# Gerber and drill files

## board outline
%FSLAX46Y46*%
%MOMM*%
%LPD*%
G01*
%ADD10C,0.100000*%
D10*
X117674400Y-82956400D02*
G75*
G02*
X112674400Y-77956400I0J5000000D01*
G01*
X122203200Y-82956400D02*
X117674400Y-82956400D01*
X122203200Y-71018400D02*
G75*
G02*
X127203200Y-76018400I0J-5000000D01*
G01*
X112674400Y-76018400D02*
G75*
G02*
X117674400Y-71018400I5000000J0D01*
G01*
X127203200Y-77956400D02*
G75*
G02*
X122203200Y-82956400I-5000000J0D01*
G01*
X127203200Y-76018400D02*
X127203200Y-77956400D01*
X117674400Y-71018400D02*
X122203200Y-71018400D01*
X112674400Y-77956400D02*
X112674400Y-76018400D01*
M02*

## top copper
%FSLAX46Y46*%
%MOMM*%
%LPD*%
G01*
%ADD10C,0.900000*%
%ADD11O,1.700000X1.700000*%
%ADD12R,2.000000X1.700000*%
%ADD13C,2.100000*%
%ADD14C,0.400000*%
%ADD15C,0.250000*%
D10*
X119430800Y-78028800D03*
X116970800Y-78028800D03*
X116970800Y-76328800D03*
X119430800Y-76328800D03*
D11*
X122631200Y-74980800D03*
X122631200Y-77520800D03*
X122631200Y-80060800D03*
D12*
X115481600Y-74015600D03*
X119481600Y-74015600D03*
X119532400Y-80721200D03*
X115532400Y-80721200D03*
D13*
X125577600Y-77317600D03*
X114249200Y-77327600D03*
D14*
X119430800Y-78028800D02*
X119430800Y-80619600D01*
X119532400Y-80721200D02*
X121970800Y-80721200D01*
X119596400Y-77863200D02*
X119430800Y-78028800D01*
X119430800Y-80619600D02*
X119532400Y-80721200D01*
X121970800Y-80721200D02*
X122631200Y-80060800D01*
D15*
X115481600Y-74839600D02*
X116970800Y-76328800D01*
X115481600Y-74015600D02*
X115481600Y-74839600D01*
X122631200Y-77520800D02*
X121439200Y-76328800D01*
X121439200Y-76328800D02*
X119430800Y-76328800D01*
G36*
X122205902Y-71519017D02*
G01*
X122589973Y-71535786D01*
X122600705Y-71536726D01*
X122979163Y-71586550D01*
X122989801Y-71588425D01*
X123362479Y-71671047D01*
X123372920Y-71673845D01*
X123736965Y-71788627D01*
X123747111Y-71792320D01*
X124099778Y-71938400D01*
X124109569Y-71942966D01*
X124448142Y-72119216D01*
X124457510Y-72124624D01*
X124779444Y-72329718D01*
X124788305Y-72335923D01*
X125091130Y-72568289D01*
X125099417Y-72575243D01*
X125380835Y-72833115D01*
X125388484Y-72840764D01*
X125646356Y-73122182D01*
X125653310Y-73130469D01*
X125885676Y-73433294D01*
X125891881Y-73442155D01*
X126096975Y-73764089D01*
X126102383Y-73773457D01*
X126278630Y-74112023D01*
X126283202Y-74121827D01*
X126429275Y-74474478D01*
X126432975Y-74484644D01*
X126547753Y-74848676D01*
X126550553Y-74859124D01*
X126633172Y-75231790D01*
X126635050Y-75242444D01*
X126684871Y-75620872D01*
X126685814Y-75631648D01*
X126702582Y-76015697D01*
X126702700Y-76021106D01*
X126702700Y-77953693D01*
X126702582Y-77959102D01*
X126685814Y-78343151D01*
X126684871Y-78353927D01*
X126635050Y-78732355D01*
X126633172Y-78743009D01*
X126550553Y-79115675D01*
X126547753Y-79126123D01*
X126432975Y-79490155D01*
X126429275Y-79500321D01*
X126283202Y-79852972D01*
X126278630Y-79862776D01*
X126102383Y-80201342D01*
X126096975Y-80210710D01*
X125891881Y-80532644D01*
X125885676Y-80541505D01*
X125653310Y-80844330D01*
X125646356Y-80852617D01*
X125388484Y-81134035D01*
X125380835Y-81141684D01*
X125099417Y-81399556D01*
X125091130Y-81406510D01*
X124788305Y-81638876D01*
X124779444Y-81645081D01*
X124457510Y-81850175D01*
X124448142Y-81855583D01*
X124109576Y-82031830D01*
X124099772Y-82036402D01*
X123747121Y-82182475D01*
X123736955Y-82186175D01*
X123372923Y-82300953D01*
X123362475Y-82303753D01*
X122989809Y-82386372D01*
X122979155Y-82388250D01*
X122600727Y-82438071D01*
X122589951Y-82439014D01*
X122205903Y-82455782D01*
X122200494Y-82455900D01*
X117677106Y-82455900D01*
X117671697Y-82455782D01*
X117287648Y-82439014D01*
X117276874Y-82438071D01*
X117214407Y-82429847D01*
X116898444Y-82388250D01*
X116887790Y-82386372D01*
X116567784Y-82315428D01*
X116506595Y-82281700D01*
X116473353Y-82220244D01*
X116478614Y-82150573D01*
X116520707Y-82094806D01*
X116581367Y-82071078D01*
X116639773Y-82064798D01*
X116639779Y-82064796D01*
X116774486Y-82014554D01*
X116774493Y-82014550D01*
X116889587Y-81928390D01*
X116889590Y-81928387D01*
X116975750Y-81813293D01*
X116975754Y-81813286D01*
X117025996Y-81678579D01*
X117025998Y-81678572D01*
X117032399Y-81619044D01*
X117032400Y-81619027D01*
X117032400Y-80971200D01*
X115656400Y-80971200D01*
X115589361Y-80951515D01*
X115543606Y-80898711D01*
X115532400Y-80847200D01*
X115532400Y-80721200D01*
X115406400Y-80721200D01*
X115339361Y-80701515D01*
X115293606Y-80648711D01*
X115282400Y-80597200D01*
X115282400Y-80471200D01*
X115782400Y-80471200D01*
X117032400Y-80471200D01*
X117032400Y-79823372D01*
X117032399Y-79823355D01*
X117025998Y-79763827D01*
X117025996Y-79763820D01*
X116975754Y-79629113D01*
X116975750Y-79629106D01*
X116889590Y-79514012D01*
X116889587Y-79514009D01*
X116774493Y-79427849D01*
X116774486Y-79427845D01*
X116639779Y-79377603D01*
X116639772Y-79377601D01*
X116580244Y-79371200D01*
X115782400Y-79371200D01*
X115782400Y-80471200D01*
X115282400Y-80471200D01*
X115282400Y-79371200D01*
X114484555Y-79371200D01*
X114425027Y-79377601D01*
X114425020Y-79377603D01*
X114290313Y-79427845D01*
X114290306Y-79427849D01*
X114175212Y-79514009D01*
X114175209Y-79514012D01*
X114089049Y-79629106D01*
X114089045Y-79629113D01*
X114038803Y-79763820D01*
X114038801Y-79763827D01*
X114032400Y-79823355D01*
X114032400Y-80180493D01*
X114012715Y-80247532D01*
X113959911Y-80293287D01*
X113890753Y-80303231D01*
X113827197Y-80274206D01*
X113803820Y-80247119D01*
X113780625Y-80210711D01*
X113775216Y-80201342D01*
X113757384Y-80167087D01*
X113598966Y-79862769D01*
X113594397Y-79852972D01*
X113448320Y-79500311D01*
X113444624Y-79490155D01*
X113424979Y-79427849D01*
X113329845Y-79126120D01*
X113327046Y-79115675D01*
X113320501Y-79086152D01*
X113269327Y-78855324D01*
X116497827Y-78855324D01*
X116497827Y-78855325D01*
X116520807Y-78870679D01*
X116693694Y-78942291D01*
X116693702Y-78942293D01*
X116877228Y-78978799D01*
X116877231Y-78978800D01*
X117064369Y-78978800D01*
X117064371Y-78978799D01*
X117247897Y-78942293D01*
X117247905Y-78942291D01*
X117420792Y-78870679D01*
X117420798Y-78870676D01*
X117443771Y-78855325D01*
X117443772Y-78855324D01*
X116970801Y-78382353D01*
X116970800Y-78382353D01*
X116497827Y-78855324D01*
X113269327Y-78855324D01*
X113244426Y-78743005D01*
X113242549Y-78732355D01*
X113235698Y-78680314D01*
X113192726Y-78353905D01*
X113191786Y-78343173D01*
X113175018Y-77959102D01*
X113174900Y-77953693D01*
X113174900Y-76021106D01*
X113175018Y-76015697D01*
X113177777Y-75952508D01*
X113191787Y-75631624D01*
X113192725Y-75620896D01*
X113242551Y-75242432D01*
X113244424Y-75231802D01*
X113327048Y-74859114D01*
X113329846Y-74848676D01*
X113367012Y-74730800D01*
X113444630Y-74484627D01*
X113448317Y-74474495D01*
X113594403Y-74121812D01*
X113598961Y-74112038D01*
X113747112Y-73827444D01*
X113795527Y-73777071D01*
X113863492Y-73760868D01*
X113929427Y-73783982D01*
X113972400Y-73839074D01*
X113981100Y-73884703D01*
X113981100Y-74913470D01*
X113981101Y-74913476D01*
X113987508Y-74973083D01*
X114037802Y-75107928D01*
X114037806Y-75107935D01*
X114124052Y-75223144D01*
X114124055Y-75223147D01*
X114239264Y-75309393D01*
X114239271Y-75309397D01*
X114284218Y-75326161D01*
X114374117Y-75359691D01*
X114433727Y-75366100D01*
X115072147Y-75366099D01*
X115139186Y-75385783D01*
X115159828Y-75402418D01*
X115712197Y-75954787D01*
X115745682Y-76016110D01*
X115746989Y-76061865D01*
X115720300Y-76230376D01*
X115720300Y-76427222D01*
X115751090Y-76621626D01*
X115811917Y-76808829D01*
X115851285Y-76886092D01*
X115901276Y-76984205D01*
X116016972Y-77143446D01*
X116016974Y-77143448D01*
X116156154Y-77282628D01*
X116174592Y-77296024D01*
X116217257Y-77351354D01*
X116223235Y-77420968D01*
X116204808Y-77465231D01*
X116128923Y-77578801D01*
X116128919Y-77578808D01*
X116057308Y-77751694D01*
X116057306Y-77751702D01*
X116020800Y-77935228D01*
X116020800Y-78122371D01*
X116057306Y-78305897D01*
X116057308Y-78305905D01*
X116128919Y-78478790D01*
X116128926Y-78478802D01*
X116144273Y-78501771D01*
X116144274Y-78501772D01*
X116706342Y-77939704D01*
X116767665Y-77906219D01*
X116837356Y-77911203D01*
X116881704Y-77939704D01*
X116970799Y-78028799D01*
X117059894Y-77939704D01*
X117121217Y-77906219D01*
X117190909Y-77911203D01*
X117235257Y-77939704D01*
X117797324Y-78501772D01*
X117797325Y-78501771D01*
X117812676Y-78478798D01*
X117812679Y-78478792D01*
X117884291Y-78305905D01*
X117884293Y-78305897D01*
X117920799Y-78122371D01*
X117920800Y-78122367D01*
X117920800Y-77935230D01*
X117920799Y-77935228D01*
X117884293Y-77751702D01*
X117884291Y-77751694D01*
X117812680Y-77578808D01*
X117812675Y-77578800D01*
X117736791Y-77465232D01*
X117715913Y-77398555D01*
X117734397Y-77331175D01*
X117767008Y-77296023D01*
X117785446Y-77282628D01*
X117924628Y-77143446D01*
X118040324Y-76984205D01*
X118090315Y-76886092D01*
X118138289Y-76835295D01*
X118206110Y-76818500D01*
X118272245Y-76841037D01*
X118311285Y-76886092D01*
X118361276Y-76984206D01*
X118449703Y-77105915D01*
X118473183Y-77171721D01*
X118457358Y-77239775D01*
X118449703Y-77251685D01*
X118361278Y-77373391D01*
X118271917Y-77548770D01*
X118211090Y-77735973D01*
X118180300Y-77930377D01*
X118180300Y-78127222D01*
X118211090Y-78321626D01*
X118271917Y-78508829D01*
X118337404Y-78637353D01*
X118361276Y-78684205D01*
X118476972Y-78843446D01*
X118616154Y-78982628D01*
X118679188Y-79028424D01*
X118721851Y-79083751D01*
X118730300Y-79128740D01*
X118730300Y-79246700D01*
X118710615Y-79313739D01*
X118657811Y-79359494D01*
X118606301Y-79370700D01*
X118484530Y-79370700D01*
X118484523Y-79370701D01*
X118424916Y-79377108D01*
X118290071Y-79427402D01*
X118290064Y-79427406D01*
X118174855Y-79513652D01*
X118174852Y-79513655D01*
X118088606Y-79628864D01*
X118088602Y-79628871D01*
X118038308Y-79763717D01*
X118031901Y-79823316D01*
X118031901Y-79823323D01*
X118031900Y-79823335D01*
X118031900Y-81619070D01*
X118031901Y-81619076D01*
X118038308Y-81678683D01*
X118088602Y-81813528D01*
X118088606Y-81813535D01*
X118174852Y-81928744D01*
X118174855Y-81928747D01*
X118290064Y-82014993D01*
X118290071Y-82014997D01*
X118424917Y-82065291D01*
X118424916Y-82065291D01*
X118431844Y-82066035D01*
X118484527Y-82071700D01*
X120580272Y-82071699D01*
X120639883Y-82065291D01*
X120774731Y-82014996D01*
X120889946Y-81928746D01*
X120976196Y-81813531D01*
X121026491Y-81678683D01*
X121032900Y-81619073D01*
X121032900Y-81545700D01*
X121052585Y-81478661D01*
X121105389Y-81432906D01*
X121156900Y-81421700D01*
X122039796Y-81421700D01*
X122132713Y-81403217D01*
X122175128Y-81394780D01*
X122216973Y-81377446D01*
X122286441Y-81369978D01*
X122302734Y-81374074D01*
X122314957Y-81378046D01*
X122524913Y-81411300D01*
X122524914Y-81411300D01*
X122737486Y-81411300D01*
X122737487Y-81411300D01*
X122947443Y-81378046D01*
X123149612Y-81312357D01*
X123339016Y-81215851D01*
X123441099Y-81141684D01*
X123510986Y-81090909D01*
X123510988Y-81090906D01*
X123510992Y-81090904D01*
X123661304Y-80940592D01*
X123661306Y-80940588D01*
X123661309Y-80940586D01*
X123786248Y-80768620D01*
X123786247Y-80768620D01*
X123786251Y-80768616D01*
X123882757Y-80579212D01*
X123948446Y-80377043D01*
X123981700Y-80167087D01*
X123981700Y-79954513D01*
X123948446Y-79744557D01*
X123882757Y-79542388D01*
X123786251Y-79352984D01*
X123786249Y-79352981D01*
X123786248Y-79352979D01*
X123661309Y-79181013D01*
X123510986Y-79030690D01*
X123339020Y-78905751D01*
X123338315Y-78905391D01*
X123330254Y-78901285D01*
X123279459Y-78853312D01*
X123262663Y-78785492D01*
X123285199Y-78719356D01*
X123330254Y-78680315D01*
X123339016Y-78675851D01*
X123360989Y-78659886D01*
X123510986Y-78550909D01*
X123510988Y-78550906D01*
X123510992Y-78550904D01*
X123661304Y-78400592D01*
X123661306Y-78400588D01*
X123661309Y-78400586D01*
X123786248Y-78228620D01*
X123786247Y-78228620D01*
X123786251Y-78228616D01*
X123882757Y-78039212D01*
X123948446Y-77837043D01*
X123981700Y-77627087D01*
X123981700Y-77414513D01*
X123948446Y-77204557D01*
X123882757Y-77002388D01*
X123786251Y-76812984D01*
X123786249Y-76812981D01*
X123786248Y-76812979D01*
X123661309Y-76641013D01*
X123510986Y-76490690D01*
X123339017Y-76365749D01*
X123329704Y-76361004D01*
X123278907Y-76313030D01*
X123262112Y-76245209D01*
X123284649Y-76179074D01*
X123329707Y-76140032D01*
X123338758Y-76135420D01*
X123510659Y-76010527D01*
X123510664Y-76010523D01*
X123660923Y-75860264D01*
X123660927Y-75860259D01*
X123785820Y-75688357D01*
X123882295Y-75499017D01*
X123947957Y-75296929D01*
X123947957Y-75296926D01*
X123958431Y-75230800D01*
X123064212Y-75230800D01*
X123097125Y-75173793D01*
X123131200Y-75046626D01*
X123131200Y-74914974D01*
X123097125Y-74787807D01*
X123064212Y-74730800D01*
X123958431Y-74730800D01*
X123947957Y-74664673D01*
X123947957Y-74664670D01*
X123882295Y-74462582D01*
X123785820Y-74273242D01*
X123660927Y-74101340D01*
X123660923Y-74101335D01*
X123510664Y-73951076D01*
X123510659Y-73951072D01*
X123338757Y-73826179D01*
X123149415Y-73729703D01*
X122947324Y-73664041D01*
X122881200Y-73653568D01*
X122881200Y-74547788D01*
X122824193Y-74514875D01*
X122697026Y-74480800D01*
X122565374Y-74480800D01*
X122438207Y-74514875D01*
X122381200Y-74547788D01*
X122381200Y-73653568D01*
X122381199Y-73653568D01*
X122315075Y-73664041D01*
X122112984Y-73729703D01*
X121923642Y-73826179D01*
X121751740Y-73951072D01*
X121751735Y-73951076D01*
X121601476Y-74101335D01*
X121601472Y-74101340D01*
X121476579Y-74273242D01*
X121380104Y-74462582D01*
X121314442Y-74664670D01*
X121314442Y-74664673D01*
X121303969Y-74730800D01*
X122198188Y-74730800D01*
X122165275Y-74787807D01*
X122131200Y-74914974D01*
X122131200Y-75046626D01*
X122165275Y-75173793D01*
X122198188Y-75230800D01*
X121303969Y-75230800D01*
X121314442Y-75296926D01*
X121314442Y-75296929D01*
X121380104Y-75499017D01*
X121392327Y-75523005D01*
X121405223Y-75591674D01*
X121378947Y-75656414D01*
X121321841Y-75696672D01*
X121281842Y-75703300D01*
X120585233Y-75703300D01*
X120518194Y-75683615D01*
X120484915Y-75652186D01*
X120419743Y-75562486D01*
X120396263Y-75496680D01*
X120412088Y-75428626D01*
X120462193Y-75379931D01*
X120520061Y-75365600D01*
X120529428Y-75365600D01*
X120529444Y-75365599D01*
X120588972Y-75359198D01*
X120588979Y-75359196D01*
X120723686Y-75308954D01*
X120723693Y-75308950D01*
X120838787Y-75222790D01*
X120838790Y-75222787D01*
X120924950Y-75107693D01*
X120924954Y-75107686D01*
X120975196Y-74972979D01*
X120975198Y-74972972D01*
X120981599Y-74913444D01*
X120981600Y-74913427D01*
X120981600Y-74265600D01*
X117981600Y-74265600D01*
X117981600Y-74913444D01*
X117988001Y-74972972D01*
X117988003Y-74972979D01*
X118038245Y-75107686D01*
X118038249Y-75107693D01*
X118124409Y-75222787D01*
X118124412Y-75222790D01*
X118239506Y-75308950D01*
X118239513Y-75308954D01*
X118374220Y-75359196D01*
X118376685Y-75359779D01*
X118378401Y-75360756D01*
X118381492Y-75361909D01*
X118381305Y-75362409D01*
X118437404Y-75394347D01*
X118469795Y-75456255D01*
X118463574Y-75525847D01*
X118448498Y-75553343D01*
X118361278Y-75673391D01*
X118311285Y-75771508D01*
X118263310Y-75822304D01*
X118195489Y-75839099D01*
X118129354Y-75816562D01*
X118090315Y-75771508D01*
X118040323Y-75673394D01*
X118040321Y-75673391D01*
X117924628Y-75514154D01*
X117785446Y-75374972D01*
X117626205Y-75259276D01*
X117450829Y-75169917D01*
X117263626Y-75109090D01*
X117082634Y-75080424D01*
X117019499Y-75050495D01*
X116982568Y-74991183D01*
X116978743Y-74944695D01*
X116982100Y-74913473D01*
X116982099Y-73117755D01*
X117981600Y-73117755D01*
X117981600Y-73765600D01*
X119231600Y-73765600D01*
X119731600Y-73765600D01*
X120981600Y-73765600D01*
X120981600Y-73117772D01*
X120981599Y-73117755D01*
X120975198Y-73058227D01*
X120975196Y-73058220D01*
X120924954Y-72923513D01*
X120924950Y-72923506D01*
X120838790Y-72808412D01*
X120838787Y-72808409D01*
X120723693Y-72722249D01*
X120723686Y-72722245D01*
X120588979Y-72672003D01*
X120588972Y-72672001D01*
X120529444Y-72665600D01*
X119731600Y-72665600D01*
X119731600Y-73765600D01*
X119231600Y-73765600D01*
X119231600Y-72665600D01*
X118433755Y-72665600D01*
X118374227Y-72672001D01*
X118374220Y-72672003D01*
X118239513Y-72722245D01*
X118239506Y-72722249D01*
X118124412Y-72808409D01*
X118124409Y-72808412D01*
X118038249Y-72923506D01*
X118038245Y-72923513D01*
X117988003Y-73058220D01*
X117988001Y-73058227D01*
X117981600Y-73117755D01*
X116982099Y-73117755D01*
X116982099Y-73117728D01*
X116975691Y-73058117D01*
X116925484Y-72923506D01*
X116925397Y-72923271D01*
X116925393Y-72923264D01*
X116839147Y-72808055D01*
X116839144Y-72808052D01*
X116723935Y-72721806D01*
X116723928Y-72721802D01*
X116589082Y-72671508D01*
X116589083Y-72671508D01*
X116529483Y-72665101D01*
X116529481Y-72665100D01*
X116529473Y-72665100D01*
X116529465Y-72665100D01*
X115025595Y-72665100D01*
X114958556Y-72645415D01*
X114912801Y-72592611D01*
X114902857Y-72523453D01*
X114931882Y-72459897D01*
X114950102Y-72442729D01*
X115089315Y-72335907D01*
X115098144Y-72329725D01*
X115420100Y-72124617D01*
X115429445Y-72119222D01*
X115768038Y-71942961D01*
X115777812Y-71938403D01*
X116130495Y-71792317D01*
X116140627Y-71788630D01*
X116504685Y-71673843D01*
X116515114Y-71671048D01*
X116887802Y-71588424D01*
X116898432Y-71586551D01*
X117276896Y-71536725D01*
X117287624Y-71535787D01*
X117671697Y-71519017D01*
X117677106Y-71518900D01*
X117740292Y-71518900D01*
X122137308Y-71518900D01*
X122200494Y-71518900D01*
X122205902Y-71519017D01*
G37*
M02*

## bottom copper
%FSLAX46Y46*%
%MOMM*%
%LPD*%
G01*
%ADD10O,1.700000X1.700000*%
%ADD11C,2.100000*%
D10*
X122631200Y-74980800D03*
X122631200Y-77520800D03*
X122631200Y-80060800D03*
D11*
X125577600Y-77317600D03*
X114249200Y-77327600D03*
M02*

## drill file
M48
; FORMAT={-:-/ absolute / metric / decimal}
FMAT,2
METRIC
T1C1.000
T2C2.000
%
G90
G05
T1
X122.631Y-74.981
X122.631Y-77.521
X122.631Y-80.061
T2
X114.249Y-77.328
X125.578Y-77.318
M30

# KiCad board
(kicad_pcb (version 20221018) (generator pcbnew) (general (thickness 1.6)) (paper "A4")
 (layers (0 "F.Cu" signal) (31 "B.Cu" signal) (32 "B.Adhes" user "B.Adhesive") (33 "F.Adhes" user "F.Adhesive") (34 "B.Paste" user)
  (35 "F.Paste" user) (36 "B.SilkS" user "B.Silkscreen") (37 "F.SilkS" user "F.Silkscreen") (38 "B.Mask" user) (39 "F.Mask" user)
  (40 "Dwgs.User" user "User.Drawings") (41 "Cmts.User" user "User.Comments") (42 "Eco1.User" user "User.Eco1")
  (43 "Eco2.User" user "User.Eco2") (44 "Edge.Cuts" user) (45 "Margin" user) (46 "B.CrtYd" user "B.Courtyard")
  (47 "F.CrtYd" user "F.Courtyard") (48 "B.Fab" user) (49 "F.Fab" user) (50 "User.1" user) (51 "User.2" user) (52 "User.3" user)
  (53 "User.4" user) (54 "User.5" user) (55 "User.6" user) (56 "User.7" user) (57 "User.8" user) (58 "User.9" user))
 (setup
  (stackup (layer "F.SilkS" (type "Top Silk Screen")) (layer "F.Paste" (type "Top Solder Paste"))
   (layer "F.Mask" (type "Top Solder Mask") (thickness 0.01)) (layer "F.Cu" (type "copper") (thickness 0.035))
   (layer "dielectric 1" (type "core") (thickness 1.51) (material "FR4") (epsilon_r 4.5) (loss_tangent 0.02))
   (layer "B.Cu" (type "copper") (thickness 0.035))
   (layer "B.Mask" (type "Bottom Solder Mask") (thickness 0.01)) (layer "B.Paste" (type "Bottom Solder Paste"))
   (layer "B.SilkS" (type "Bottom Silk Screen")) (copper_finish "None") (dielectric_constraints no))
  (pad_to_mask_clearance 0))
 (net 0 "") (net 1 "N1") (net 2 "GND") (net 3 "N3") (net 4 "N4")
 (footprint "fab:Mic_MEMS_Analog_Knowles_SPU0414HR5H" (layer "F.Cu") (at 118.2008 77.1788 -90) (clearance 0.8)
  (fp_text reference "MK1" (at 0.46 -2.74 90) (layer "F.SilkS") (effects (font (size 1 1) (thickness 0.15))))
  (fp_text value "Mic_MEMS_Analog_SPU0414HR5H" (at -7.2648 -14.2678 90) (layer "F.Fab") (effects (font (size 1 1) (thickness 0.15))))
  (pad "1" smd circle (at 0.85 -1.23 270) (size 0.9 0.9) (layers "F.Cu" "F.Paste" "F.Mask") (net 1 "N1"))
  (pad "2" smd circle (at 0.85 1.23 270) (size 0.9 0.9) (layers "F.Cu" "F.Paste" "F.Mask") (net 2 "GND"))
  (pad "3" smd circle (at -0.85 1.23 270) (size 0.9 0.9) (layers "F.Cu" "F.Paste" "F.Mask") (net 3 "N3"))
  (pad "4" smd circle (at -0.85 -1.23 270) (size 0.9 0.9) (layers "F.Cu" "F.Paste" "F.Mask") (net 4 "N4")))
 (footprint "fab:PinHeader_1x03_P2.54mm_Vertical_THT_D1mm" (layer "F.Cu") (at 122.6312 74.9808)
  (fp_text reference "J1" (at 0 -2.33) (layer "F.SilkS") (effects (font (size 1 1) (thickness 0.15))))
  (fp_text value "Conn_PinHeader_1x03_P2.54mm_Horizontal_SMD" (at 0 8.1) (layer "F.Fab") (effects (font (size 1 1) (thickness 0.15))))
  (pad "1" thru_hole oval (at 0 0) (size 1.7 1.7) (drill 1) (layers "*.Cu" "*.Mask") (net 2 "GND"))
  (pad "2" thru_hole oval (at 0 2.54) (size 1.7 1.7) (drill 1) (layers "*.Cu" "*.Mask") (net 4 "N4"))
  (pad "3" thru_hole oval (at 0 5.08) (size 1.7 1.7) (drill 1) (layers "*.Cu" "*.Mask") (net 1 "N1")))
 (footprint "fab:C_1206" (layer "F.Cu") (at 117.4816 74.0156)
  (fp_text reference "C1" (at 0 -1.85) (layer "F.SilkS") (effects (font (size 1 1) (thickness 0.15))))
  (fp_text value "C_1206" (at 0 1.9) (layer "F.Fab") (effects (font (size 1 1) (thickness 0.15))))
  (pad "1" smd rect (at -2 0) (size 2 1.7) (layers "F.Cu" "F.Paste" "F.Mask") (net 3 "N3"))
  (pad "2" smd rect (at 2 0) (size 2 1.7) (layers "F.Cu" "F.Paste" "F.Mask") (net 2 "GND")))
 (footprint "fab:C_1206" (layer "F.Cu") (at 117.5324 80.7212 180)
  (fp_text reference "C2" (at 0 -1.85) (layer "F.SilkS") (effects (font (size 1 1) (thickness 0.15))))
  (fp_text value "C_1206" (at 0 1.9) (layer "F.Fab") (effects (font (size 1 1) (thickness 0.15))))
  (pad "1" smd rect (at -2 0 180) (size 2 1.7) (layers "F.Cu" "F.Paste" "F.Mask") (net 1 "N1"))
  (pad "2" smd rect (at 2 0 180) (size 2 1.7) (layers "F.Cu" "F.Paste" "F.Mask") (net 2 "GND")))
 (gr_arc (start 117.6744 82.9564) (mid 114.138866 81.491934) (end 112.6744 77.9564) (stroke (width 0.1) (type default)) (layer "Edge.Cuts"))
 (gr_line (start 122.2032 82.9564) (end 117.6744 82.9564) (stroke (width 0.1) (type default)) (layer "Edge.Cuts"))
 (gr_arc (start 122.2032 71.0184) (mid 125.738734 72.482866) (end 127.2032 76.0184) (stroke (width 0.1) (type default)) (layer "Edge.Cuts"))
 (gr_arc (start 112.6744 76.0184) (mid 114.138866 72.482866) (end 117.6744 71.0184) (stroke (width 0.1) (type default)) (layer "Edge.Cuts"))
 (gr_arc (start 127.2032 77.9564) (mid 125.738734 81.491934) (end 122.2032 82.9564) (stroke (width 0.1) (type default)) (layer "Edge.Cuts"))
 (gr_line (start 127.2032 76.0184) (end 127.2032 77.9564) (stroke (width 0.1) (type default)) (layer "Edge.Cuts"))
 (gr_line (start 117.6744 71.0184) (end 122.2032 71.0184) (stroke (width 0.1) (type default)) (layer "Edge.Cuts"))
 (gr_line (start 112.6744 77.9564) (end 112.6744 76.0184) (stroke (width 0.1) (type default)) (layer "Edge.Cuts"))
 (via (at 125.5776 77.3176) (size 2.1) (drill 2) (layers "F.Cu" "B.Cu") (free) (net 2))
 (via (at 114.2492 77.3276) (size 2.1) (drill 2) (layers "F.Cu" "B.Cu") (free) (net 2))
 (segment (start 119.4308 78.0288) (end 119.4308 80.6196) (width 0.4) (layer "F.Cu") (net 1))
 (segment (start 119.5324 80.7212) (end 121.9708 80.7212) (width 0.4) (layer "F.Cu") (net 1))
 (segment (start 119.5964 77.8632) (end 119.4308 78.0288) (width 0.4) (layer "F.Cu") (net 1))
 (segment (start 119.4308 80.6196) (end 119.5324 80.7212) (width 0.4) (layer "F.Cu") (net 1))
 (segment (start 121.9708 80.7212) (end 122.6312 80.0608) (width 0.4) (layer "F.Cu") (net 1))
 (segment (start 115.4816 74.8396) (end 116.9708 76.3288) (width 0.25) (layer "F.Cu") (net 3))
 (segment (start 115.4816 74.0156) (end 115.4816 74.8396) (width 0.25) (layer "F.Cu") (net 3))
 (segment (start 122.6312 77.5208) (end 121.4392 76.3288) (width 0.25) (layer "F.Cu") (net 4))
 (segment (start 121.4392 76.3288) (end 119.4308 76.3288) (width 0.25) (layer "F.Cu") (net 4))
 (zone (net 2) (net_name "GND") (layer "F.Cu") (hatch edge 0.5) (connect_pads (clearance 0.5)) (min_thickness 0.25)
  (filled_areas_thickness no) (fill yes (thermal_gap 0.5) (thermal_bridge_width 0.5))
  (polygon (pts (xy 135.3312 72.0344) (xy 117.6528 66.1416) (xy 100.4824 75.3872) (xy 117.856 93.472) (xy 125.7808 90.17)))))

